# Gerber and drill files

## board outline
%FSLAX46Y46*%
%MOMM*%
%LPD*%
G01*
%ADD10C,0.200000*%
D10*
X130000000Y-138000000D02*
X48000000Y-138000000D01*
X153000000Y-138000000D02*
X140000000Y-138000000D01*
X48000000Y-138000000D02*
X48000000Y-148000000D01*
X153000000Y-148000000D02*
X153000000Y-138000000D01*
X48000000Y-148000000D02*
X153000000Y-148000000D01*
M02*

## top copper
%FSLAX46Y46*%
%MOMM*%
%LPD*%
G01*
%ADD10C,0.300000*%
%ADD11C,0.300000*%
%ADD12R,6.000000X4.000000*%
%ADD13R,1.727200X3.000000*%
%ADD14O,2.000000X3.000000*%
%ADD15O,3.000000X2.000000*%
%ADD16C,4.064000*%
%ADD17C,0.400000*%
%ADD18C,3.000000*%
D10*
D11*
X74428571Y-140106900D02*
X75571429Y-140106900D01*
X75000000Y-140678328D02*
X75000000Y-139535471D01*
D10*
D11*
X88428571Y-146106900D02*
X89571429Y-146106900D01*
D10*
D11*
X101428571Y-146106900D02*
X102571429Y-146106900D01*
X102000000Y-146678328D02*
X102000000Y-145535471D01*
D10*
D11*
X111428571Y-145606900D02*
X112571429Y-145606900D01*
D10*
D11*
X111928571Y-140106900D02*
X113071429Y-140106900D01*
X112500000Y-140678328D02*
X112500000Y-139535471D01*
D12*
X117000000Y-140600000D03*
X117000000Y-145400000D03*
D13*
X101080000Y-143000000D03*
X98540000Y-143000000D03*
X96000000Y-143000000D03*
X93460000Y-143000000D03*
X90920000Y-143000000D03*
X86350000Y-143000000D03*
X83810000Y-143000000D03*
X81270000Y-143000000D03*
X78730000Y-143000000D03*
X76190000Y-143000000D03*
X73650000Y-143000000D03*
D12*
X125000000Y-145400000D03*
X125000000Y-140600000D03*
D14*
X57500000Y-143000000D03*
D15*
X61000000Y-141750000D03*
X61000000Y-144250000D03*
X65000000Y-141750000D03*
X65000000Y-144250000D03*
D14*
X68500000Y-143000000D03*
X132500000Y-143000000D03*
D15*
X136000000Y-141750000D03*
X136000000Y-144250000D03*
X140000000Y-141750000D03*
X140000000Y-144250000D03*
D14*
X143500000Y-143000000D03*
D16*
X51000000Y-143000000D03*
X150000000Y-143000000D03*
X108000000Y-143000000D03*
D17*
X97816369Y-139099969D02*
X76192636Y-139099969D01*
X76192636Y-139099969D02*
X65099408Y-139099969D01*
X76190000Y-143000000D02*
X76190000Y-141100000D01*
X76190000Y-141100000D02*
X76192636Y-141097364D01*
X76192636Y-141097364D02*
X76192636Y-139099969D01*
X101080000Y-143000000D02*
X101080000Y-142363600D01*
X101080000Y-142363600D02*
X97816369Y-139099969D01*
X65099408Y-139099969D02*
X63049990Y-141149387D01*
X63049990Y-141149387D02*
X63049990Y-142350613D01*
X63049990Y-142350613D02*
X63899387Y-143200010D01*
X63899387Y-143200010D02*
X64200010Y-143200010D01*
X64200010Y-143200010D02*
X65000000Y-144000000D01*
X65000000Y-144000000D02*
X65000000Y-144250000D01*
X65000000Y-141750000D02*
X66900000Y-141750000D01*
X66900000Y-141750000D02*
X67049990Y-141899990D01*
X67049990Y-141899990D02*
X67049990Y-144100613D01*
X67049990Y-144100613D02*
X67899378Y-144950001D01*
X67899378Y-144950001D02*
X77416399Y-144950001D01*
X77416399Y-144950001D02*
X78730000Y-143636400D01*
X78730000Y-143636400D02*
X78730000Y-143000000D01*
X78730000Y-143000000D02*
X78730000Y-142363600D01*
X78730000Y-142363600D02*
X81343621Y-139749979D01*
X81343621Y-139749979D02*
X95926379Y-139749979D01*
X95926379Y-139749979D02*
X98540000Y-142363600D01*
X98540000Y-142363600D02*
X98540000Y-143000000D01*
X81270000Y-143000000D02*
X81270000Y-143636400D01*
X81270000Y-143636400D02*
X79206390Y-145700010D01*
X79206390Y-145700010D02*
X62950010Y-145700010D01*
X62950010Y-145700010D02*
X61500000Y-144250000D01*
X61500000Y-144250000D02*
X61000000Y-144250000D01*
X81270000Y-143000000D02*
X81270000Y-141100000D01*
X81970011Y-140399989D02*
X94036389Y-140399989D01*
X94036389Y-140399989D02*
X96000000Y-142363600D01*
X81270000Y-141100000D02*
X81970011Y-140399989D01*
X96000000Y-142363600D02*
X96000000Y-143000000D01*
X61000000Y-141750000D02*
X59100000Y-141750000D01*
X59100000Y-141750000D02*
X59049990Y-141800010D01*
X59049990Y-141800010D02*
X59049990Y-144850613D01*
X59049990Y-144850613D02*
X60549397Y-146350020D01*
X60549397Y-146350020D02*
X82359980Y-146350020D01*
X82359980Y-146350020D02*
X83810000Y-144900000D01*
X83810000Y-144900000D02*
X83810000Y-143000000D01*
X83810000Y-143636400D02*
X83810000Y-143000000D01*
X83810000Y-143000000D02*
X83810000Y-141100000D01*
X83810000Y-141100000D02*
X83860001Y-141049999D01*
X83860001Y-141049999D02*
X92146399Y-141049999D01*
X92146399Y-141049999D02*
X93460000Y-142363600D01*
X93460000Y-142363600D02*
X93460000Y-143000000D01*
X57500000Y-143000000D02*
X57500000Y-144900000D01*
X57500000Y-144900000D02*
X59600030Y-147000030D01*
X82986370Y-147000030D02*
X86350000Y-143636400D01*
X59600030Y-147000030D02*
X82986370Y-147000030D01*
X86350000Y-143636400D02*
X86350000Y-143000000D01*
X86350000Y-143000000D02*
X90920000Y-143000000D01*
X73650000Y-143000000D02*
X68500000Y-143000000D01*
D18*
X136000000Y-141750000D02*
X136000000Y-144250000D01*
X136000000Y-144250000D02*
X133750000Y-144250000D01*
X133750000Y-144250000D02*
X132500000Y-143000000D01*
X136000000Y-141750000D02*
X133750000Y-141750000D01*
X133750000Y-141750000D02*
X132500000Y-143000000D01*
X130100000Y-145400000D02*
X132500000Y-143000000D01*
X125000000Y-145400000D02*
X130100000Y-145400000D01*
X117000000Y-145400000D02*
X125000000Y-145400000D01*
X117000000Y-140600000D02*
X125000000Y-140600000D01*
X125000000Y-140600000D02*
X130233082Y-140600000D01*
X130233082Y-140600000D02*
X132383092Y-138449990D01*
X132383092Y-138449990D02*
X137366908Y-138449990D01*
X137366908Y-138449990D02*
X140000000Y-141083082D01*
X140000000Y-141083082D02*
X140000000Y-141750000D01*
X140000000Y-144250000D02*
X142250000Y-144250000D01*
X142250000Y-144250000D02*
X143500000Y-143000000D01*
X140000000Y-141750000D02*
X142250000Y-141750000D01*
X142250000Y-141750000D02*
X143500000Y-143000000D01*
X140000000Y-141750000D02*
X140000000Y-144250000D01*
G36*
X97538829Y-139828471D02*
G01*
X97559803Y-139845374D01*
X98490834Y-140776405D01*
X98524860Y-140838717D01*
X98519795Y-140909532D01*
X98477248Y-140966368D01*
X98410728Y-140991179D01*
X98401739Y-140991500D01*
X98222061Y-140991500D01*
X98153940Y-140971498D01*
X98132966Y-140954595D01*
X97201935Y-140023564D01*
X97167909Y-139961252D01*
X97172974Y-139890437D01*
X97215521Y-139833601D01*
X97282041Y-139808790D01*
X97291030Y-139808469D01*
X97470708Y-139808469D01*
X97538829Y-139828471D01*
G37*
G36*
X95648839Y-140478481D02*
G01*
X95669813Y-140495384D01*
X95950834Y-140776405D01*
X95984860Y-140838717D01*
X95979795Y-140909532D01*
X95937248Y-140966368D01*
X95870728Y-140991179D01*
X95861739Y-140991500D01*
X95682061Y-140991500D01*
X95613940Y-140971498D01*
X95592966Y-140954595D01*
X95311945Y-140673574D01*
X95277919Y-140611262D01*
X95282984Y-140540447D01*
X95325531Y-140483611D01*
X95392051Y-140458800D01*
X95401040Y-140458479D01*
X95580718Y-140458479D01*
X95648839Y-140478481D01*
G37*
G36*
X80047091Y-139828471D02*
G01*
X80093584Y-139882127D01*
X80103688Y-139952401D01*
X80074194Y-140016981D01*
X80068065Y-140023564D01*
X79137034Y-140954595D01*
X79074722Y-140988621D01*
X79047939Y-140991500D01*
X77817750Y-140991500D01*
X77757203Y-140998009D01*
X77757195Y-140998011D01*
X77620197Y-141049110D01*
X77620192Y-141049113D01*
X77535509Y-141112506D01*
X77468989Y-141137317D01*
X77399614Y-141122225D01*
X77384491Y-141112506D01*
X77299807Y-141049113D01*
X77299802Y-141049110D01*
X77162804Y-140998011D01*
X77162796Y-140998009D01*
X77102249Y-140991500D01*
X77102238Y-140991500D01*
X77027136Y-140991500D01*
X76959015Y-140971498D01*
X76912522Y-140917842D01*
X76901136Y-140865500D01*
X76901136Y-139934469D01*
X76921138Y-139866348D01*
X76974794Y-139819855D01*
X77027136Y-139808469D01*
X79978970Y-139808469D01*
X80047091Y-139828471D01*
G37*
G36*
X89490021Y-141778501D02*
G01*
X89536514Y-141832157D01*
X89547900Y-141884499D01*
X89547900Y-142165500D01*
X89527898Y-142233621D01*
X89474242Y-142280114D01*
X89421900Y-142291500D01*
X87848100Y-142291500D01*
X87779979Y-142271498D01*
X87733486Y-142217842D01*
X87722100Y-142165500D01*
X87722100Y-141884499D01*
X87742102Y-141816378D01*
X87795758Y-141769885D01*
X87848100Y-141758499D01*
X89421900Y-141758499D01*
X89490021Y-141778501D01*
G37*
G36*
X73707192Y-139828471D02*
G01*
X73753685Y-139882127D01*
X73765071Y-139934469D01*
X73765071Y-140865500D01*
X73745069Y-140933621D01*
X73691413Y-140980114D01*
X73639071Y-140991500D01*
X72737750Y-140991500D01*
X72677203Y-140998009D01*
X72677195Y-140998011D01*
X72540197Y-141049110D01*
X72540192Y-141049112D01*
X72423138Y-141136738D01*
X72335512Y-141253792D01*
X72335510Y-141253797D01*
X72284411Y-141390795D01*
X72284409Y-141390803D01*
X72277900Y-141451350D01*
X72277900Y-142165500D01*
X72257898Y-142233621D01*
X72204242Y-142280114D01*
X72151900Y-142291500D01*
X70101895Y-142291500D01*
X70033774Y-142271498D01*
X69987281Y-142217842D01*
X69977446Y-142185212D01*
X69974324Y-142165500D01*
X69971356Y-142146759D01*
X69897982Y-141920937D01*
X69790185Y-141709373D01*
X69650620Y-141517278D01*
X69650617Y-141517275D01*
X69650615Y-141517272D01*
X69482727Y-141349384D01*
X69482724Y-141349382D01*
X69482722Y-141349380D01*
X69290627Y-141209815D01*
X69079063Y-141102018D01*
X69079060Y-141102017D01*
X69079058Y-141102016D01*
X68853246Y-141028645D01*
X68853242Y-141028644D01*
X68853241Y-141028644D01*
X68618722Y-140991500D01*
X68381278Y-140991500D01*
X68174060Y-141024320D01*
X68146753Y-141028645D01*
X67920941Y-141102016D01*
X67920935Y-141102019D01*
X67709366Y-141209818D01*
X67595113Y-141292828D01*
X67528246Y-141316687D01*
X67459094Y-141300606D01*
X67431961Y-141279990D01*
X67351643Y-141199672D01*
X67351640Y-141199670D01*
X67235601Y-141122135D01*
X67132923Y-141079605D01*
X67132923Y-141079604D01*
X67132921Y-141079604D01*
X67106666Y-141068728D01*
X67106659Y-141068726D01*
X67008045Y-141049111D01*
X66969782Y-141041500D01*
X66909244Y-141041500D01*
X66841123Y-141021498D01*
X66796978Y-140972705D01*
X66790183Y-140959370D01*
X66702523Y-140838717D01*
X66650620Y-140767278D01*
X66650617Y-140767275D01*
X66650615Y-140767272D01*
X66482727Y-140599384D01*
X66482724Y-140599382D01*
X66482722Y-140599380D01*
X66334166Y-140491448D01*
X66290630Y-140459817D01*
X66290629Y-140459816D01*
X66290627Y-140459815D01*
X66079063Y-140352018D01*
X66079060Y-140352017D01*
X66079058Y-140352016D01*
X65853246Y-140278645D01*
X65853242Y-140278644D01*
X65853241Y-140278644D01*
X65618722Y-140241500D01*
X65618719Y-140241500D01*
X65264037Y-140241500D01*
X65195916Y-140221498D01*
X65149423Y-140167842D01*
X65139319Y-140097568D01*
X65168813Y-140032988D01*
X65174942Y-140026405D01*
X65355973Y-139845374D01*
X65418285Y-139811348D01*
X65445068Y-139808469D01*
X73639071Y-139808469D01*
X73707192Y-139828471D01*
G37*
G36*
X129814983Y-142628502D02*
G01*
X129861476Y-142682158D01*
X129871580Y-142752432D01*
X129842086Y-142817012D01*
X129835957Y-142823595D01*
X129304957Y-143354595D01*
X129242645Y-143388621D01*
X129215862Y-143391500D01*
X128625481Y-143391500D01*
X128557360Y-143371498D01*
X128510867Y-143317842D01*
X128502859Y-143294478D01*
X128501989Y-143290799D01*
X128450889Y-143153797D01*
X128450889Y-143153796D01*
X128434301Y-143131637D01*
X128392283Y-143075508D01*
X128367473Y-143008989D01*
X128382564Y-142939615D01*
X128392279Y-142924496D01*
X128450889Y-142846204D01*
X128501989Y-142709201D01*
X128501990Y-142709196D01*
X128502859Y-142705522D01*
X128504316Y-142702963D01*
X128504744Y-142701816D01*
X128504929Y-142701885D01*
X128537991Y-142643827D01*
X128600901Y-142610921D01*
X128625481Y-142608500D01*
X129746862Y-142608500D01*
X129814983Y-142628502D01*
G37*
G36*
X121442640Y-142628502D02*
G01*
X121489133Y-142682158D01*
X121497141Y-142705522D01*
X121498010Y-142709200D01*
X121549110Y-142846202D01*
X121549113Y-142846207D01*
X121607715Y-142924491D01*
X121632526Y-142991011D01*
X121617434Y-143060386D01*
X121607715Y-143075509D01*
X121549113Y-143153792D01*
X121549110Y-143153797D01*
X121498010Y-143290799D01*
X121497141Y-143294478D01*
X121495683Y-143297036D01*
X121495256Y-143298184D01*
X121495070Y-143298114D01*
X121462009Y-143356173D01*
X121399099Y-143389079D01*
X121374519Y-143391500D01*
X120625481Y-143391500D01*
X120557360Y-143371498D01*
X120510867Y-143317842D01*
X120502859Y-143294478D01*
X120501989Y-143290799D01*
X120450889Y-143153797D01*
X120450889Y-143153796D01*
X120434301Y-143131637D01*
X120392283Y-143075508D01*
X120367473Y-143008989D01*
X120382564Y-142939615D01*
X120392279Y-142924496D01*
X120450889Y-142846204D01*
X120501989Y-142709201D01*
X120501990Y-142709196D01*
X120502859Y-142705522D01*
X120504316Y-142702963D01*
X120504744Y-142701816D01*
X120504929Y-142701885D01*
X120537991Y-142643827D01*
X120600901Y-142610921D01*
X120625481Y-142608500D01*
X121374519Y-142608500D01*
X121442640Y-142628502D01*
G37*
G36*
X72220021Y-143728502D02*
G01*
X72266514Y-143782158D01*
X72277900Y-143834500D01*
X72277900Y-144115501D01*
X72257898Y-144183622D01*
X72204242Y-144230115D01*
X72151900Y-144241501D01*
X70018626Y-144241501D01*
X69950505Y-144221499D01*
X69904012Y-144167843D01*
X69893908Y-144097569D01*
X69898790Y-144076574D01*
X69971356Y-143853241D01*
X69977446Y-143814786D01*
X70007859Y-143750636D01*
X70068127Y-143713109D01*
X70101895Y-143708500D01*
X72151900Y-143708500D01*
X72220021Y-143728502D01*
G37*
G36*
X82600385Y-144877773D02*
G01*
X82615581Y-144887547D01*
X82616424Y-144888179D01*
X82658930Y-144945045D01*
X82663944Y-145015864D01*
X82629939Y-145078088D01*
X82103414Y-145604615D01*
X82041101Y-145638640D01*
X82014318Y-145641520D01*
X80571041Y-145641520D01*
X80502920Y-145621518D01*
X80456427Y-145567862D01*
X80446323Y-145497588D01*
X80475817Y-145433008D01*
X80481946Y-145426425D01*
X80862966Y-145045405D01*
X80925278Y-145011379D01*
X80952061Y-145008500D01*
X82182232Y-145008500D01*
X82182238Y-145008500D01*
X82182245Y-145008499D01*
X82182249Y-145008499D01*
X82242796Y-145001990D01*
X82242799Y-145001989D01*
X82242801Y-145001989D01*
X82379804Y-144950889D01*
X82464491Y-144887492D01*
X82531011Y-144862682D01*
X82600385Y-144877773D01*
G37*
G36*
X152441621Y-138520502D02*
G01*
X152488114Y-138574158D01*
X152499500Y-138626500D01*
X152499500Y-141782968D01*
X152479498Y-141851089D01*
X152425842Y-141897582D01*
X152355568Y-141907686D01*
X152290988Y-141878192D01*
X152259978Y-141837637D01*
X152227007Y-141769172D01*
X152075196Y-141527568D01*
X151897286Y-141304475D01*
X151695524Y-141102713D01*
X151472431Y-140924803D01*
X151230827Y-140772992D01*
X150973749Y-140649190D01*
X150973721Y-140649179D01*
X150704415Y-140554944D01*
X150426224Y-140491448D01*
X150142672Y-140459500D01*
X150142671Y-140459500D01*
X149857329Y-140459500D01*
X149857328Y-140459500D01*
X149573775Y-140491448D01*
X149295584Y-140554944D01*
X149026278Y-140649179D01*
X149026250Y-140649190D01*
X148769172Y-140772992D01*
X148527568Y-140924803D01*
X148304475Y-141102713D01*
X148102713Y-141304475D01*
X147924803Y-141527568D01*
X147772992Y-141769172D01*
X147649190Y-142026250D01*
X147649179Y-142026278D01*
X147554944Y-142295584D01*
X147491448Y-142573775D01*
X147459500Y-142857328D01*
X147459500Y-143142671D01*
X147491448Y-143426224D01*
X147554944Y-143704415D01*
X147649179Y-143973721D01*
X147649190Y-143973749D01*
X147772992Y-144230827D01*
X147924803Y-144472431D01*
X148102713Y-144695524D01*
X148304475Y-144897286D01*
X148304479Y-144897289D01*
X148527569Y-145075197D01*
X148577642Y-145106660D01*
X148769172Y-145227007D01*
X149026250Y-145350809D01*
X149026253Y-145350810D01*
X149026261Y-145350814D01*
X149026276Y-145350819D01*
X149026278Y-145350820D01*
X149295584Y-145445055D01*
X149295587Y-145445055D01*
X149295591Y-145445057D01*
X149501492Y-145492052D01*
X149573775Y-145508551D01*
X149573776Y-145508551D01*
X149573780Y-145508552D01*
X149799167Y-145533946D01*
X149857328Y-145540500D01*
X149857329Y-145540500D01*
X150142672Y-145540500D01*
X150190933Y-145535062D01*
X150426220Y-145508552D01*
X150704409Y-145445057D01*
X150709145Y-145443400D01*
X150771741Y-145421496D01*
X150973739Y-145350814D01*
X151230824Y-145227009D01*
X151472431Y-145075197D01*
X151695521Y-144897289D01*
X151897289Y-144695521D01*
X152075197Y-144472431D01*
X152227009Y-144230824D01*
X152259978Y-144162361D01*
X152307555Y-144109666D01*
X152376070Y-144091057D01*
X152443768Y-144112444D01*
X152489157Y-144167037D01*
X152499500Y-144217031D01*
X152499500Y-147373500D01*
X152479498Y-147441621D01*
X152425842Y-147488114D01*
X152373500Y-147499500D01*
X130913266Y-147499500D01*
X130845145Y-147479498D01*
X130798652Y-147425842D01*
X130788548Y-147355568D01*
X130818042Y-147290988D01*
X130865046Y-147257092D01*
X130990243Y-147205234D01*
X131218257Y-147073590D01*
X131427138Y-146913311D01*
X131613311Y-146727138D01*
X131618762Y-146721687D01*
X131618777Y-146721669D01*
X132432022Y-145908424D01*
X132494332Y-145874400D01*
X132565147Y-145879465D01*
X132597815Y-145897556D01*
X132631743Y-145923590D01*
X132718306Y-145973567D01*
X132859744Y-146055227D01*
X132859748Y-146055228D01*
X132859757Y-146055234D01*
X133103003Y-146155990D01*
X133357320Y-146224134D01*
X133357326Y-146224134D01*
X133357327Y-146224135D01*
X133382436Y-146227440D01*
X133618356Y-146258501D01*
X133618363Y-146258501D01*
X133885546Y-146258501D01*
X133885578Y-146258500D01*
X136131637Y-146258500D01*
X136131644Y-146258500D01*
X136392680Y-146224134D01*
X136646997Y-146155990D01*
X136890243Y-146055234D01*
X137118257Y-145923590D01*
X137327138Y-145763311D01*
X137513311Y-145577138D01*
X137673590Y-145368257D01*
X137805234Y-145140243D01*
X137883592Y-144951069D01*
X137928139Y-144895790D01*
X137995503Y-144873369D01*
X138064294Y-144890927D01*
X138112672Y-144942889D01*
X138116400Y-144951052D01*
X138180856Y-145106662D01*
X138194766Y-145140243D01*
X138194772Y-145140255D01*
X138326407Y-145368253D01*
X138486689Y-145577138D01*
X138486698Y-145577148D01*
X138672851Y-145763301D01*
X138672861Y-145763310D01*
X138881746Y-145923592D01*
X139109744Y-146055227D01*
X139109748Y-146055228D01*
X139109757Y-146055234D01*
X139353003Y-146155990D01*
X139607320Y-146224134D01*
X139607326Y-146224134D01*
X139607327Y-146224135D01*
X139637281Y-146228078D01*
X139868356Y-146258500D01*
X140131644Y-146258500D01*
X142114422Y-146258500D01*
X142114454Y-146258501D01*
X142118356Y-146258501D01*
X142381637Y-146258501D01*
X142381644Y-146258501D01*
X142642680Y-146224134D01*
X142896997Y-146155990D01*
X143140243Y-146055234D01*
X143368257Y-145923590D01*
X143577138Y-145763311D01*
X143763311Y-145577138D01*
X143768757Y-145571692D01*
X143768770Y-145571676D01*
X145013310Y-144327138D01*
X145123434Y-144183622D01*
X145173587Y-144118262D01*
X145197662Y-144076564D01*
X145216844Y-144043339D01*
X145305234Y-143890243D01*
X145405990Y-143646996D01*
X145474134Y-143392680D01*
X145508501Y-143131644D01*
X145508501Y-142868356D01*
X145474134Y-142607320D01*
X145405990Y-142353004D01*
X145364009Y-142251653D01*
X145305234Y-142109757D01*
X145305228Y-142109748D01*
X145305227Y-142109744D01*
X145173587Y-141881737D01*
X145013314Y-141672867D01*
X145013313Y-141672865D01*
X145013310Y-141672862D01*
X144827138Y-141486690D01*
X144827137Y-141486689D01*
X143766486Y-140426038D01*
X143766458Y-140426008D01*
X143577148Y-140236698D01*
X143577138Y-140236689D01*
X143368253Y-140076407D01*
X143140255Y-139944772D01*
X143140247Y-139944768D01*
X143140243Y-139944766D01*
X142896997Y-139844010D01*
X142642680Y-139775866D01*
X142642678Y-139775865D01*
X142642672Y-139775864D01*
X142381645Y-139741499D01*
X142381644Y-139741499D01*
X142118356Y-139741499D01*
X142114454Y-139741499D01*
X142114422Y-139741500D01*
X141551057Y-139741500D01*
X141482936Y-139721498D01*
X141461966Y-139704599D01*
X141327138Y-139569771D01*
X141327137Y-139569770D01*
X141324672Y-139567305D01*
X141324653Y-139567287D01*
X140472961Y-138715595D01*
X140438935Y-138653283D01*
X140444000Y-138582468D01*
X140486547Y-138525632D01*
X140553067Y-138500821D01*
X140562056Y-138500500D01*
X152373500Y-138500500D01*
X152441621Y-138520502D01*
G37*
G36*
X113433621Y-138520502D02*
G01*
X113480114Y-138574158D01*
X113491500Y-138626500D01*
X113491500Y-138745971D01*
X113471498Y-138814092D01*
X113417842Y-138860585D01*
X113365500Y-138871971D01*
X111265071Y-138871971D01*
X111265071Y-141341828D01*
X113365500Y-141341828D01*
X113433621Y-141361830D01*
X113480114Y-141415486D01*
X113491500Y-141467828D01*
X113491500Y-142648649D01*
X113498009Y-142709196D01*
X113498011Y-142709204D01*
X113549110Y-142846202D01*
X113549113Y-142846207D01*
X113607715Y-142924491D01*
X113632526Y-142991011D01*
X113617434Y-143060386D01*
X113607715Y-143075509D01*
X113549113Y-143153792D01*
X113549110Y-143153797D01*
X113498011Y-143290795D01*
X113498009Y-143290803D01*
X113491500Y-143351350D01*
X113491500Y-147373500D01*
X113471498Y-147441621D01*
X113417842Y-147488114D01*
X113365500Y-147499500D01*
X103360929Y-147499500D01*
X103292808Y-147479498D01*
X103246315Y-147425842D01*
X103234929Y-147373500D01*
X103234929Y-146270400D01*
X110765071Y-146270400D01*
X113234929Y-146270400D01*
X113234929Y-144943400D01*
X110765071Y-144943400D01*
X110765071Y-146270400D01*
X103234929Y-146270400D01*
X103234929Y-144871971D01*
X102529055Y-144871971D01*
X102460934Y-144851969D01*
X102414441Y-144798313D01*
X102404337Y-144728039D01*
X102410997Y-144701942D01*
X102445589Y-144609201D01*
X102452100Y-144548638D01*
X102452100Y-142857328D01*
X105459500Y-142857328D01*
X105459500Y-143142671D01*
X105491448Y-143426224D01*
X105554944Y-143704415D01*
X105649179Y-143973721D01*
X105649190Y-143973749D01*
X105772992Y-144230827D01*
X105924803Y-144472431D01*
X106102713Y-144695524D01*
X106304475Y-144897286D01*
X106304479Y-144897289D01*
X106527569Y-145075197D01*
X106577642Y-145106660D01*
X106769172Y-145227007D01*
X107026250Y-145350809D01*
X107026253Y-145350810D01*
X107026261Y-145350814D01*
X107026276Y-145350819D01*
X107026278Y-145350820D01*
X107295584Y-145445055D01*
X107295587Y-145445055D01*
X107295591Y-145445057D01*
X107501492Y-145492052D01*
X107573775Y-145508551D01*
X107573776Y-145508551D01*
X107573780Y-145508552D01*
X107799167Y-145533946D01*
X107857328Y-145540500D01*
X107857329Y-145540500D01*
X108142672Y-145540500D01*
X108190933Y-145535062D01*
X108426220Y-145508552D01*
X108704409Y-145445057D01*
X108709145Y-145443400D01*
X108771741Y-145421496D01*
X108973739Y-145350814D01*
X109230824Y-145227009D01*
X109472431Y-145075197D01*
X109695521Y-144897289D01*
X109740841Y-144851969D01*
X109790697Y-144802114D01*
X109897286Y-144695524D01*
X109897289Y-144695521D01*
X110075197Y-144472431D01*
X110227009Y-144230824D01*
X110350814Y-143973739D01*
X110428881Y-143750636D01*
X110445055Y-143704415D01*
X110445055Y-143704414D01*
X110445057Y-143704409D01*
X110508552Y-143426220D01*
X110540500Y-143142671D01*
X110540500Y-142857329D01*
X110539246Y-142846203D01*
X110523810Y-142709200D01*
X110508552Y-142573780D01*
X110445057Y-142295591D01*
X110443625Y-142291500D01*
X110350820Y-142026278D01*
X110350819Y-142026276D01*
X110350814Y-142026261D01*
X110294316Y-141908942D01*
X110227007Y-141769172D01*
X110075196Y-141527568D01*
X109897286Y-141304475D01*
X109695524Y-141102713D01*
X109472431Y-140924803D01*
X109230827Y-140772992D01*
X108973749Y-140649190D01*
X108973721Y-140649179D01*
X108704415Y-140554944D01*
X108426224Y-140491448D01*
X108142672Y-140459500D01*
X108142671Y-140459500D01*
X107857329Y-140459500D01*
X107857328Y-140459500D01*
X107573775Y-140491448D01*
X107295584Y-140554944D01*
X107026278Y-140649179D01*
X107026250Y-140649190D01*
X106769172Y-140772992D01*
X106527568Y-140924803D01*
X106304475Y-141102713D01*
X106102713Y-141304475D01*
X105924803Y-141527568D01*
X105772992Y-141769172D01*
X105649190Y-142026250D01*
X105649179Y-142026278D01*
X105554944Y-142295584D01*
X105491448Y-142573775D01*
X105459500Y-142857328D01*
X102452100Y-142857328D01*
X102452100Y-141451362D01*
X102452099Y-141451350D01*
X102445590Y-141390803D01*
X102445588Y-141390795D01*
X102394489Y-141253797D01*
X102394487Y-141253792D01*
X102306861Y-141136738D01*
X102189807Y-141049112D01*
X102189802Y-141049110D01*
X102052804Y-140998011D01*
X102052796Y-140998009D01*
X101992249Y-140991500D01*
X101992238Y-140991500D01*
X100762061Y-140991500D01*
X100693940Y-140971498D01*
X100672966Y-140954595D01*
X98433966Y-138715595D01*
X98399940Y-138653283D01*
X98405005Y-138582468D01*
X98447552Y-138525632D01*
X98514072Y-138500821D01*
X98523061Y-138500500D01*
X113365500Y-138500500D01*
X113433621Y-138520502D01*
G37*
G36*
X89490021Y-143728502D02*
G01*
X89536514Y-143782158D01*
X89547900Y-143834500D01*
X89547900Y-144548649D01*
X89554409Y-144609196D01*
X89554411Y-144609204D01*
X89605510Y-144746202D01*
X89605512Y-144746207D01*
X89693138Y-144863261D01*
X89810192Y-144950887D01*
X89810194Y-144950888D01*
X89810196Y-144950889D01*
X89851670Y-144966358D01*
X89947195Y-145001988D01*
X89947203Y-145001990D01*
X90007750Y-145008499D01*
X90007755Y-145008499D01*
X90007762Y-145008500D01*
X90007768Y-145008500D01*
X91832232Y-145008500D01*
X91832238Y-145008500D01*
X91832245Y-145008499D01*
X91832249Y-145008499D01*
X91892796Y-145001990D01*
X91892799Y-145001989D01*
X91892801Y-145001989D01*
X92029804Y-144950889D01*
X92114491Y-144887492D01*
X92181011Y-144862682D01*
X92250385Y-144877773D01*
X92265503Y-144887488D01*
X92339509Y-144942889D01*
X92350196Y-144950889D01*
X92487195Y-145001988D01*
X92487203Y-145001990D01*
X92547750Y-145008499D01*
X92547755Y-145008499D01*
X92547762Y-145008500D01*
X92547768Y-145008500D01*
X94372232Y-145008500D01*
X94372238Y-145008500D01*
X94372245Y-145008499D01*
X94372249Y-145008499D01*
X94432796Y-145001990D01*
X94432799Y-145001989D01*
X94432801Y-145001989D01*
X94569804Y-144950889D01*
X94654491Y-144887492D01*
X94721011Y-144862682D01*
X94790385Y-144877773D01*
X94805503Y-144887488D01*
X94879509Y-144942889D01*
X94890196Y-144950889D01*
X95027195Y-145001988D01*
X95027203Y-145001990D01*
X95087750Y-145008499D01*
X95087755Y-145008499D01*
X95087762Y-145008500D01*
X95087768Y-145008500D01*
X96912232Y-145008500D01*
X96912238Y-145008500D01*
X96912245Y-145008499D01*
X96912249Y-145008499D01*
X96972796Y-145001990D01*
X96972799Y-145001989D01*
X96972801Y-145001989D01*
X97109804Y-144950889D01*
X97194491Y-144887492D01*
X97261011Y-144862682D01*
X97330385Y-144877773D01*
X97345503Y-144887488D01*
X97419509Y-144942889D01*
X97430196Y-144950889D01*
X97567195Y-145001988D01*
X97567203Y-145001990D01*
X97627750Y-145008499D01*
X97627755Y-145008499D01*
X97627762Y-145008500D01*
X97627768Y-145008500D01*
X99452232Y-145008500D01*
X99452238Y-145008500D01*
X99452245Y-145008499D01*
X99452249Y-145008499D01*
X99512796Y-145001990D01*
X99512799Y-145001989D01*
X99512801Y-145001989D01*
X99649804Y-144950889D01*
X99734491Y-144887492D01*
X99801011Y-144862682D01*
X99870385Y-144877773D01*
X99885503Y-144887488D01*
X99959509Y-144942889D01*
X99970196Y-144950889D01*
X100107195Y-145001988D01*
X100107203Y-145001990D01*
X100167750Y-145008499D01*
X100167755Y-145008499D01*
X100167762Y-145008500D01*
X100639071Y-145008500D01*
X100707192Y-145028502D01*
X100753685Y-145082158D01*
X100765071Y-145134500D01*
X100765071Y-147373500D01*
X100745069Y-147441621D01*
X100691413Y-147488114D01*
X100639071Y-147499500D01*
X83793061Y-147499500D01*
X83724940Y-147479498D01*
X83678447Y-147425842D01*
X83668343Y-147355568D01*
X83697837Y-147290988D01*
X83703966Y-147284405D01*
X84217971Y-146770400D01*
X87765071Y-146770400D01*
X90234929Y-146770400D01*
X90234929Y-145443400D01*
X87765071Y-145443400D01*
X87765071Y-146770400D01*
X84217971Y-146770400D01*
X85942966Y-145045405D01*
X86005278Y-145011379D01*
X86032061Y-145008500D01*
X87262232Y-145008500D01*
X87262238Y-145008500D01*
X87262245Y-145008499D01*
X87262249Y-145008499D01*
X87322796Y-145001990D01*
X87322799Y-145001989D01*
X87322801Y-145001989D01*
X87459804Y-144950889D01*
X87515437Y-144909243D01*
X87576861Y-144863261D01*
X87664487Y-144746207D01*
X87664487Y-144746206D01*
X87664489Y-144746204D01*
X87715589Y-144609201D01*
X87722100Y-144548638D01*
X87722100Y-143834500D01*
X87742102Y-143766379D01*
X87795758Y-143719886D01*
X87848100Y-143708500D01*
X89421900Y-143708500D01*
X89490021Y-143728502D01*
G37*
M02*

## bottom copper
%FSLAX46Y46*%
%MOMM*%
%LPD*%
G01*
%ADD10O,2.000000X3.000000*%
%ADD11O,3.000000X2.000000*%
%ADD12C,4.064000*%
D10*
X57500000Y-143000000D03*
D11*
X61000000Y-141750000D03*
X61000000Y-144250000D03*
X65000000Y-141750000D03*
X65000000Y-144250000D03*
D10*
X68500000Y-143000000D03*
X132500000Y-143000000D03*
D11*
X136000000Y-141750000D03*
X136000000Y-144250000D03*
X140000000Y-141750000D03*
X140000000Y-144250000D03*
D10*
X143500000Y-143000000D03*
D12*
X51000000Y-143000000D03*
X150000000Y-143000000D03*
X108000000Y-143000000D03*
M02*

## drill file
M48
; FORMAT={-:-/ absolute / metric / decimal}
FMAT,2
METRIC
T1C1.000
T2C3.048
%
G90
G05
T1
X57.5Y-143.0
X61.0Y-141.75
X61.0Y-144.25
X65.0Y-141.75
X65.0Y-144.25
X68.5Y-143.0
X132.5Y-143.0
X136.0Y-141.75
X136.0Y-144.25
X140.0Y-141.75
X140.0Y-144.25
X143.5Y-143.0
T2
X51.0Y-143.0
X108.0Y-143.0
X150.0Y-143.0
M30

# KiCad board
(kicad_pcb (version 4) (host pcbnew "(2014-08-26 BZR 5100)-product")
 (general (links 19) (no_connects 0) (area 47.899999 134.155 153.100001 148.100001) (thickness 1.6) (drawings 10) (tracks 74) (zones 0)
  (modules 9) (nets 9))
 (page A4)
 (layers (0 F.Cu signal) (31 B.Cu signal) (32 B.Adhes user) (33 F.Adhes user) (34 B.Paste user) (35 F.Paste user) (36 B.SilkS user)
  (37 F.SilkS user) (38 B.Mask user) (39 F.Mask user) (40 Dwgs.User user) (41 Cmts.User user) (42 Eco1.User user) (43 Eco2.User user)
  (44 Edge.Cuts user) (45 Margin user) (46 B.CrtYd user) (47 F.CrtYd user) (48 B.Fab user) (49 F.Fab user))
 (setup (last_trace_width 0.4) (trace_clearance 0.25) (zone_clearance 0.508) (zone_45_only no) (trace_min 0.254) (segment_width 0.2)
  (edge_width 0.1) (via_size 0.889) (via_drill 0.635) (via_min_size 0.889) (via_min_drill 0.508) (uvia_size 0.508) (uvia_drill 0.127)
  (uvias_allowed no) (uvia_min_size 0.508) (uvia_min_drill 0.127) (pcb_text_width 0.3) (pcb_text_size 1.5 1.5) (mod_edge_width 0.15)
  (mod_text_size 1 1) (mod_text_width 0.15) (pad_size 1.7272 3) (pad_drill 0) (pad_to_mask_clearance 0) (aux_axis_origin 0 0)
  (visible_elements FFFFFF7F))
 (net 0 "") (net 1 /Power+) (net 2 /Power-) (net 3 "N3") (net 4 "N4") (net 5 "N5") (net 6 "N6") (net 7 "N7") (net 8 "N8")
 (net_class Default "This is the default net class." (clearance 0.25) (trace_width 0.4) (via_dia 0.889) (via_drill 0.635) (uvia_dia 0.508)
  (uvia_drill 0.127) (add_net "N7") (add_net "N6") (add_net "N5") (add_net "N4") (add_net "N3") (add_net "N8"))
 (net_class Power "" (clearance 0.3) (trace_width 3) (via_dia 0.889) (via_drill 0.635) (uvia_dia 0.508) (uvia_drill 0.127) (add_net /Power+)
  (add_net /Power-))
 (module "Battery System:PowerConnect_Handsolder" (layer F.Cu) (at 117 143)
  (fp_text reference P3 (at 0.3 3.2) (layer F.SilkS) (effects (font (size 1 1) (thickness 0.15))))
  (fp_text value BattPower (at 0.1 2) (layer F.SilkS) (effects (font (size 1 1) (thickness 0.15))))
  (pad 1 smd rect (at 0 -2.4) (size 6 4) (layers F.Cu F.Paste F.Mask) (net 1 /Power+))
  (pad 2 smd rect (at 0 2.4) (size 6 4) (layers F.Cu F.Paste F.Mask) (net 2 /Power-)))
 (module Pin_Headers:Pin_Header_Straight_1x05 (layer F.Cu) (at 96 143 180)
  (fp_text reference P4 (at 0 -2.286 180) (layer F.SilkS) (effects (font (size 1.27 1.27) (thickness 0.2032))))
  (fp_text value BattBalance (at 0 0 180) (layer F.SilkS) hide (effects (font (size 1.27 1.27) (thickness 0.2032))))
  (pad 1 smd rect (at -5.08 0) (size 1.7272 3) (layers F.Cu F.Paste F.Mask) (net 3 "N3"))
  (pad 2 smd rect (at -2.54 0) (size 1.7272 3) (layers F.Cu F.Paste F.Mask) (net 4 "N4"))
  (pad 3 smd rect (at 0 0) (size 1.7272 3) (layers F.Cu F.Paste F.Mask) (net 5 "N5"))
  (pad 4 smd rect (at 2.54 0) (size 1.7272 3) (layers F.Cu F.Paste F.Mask) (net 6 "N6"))
  (pad 5 smd rect (at 5.08 0) (size 1.7272 3) (layers F.Cu F.Paste F.Mask) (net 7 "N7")))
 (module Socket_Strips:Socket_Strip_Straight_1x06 (layer F.Cu) (at 80 143)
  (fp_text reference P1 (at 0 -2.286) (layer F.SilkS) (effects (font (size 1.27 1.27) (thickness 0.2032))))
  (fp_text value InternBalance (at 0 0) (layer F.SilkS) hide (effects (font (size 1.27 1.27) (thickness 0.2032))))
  (pad 1 smd rect (at 6.35 0 180) (size 1.7272 3) (layers F.Cu F.Paste F.Mask) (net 7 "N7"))
  (pad 2 smd rect (at 3.81 0 180) (size 1.7272 3) (layers F.Cu F.Paste F.Mask) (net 6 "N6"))
  (pad 3 smd rect (at 1.27 0 180) (size 1.7272 3) (layers F.Cu F.Paste F.Mask) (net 5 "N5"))
  (pad 4 smd rect (at -1.27 0 180) (size 1.7272 3) (layers F.Cu F.Paste F.Mask) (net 4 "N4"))
  (pad 5 smd rect (at -3.81 0 180) (size 1.7272 3) (layers F.Cu F.Paste F.Mask) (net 3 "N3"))
  (pad 6 smd rect (at -6.35 0 180) (size 1.7272 3) (layers F.Cu F.Paste F.Mask) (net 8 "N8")))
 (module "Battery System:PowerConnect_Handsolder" (layer F.Cu) (at 125 143 180)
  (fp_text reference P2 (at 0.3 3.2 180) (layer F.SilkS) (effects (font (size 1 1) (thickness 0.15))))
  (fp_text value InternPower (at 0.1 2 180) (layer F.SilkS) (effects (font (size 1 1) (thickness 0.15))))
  (pad 1 smd rect (at 0 -2.4 180) (size 6 4) (layers F.Cu F.Paste F.Mask) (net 2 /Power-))
  (pad 2 smd rect (at 0 2.4 180) (size 6 4) (layers F.Cu F.Paste F.Mask) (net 1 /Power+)))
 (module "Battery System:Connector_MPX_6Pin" (layer B.Cu) (at 63 143)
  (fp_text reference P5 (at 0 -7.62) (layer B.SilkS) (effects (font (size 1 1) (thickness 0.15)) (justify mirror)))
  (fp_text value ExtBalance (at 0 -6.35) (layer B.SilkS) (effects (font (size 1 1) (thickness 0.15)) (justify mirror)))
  (pad 1 thru_hole oval (at -5.5 0 180) (size 2 3) (drill 1) (layers *.Cu *.Mask B.SilkS) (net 7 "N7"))
  (pad 2 thru_hole oval (at -2 -1.25 180) (size 3 2) (drill 1) (layers *.Cu *.Mask B.SilkS) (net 6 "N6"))
  (pad 3 thru_hole oval (at -2 1.25 180) (size 3 2) (drill 1) (layers *.Cu *.Mask B.SilkS) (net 5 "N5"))
  (pad 4 thru_hole oval (at 2 -1.25 180) (size 3 2) (drill 1) (layers *.Cu *.Mask B.SilkS) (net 4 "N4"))
  (pad 5 thru_hole oval (at 2 1.25 180) (size 3 2) (drill 1) (layers *.Cu *.Mask B.SilkS) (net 3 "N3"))
  (pad 6 thru_hole oval (at 5.5 0 180) (size 2 3) (drill 1) (layers *.Cu *.Mask B.SilkS) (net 8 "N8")))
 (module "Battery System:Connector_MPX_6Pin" (layer B.Cu) (at 138 143)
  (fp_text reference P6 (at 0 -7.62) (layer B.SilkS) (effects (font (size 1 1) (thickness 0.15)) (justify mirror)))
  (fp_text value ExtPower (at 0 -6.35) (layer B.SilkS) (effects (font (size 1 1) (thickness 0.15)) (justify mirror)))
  (pad 1 thru_hole oval (at -5.5 0 180) (size 2 3) (drill 1) (layers *.Cu *.Mask B.SilkS) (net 2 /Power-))
  (pad 2 thru_hole oval (at -2 -1.25 180) (size 3 2) (drill 1) (layers *.Cu *.Mask B.SilkS) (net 2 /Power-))
  (pad 3 thru_hole oval (at -2 1.25 180) (size 3 2) (drill 1) (layers *.Cu *.Mask B.SilkS) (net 2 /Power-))
  (pad 4 thru_hole oval (at 2 -1.25 180) (size 3 2) (drill 1) (layers *.Cu *.Mask B.SilkS) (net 1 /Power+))
  (pad 5 thru_hole oval (at 2 1.25 180) (size 3 2) (drill 1) (layers *.Cu *.Mask B.SilkS) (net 1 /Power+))
  (pad 6 thru_hole oval (at 5.5 0 180) (size 2 3) (drill 1) (layers *.Cu *.Mask B.SilkS) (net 1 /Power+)))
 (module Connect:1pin (layer F.Cu) (at 51 143)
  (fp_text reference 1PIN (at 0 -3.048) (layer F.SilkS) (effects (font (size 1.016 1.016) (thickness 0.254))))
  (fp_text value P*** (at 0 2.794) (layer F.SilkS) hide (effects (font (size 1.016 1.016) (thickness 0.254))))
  (pad 1 thru_hole circle (at 0 0) (size 4.064 4.064) (drill 3.048) (layers *.Cu *.Mask F.SilkS)))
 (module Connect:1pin (layer F.Cu) (at 150 143)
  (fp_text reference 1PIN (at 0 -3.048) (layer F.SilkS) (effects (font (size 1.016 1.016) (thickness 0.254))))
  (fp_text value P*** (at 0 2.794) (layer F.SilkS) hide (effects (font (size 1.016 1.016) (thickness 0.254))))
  (pad 1 thru_hole circle (at 0 0) (size 4.064 4.064) (drill 3.048) (layers *.Cu *.Mask F.SilkS)))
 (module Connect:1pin (layer F.Cu) (at 108 143)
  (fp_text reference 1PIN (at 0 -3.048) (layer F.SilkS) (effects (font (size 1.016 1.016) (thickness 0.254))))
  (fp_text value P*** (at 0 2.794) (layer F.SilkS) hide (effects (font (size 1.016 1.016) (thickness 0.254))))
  (pad 1 thru_hole circle (at 0 0) (size 4.064 4.064) (drill 3.048) (layers *.Cu *.Mask F.SilkS)))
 (gr_line (start 130 138) (end 48 138) (layer Edge.Cuts) (width 0.2))
 (gr_line (start 153 138) (end 140 138) (layer Edge.Cuts) (width 0.2))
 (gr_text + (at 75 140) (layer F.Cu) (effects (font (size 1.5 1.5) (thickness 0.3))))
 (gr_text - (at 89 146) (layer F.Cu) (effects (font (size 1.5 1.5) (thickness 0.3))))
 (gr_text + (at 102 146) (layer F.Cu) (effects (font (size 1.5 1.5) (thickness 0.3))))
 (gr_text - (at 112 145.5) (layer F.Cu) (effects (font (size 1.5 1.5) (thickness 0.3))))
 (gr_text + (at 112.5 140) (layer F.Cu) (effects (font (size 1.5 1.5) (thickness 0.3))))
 (gr_line (start 48 138) (end 48 148) (layer Edge.Cuts) (width 0.2))
 (gr_line (start 153 148) (end 153 138) (layer Edge.Cuts) (width 0.2))
 (gr_line (start 48 148) (end 153 148) (layer Edge.Cuts) (width 0.2))
 (segment (start 97.816369 139.099969) (end 76.192636 139.099969) (width 0.4) (layer F.Cu) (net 3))
 (segment (start 76.192636 139.099969) (end 65.099408 139.099969) (width 0.4) (layer F.Cu) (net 3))
 (segment (start 76.19 143) (end 76.19 141.1) (width 0.4) (layer F.Cu) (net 3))
 (segment (start 76.19 141.1) (end 76.192636 141.097364) (width 0.4) (layer F.Cu) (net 3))
 (segment (start 76.192636 141.097364) (end 76.192636 139.099969) (width 0.4) (layer F.Cu) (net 3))
 (segment (start 101.08 143) (end 101.08 142.3636) (width 0.4) (layer F.Cu) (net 3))
 (segment (start 101.08 142.3636) (end 97.816369 139.099969) (width 0.4) (layer F.Cu) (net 3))
 (segment (start 65.099408 139.099969) (end 63.04999 141.149387) (width 0.4) (layer F.Cu) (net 3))
 (segment (start 63.04999 141.149387) (end 63.04999 142.350613) (width 0.4) (layer F.Cu) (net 3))
 (segment (start 63.04999 142.350613) (end 63.899387 143.20001) (width 0.4) (layer F.Cu) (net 3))
 (segment (start 63.899387 143.20001) (end 64.20001 143.20001) (width 0.4) (layer F.Cu) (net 3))
 (segment (start 64.20001 143.20001) (end 65 144) (width 0.4) (layer F.Cu) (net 3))
 (segment (start 65 144) (end 65 144.25) (width 0.4) (layer F.Cu) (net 3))
 (segment (start 65 141.75) (end 66.9 141.75) (width 0.4) (layer F.Cu) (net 4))
 (segment (start 66.9 141.75) (end 67.04999 141.89999) (width 0.4) (layer F.Cu) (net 4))
 (segment (start 67.04999 141.89999) (end 67.04999 144.100613) (width 0.4) (layer F.Cu) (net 4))
 (segment (start 67.04999 144.100613) (end 67.899378 144.950001) (width 0.4) (layer F.Cu) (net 4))
 (segment (start 67.899378 144.950001) (end 77.416399 144.950001) (width 0.4) (layer F.Cu) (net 4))
 (segment (start 77.416399 144.950001) (end 78.73 143.6364) (width 0.4) (layer F.Cu) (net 4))
 (segment (start 78.73 143.6364) (end 78.73 143) (width 0.4) (layer F.Cu) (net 4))
 (segment (start 78.73 143) (end 78.73 142.3636) (width 0.4) (layer F.Cu) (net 4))
 (segment (start 78.73 142.3636) (end 81.343621 139.749979) (width 0.4) (layer F.Cu) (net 4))
 (segment (start 81.343621 139.749979) (end 95.926379 139.749979) (width 0.4) (layer F.Cu) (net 4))
 (segment (start 95.926379 139.749979) (end 98.54 142.3636) (width 0.4) (layer F.Cu) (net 4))
 (segment (start 98.54 142.3636) (end 98.54 143) (width 0.4) (layer F.Cu) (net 4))
 (segment (start 81.27 143) (end 81.27 143.6364) (width 0.4) (layer F.Cu) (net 5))
 (segment (start 81.27 143.6364) (end 79.20639 145.70001) (width 0.4) (layer F.Cu) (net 5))
 (segment (start 79.20639 145.70001) (end 62.95001 145.70001) (width 0.4) (layer F.Cu) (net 5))
 (segment (start 62.95001 145.70001) (end 61.5 144.25) (width 0.4) (layer F.Cu) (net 5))
 (segment (start 61.5 144.25) (end 61 144.25) (width 0.4) (layer F.Cu) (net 5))
 (segment (start 81.27 143) (end 81.27 141.1) (width 0.4) (layer F.Cu) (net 5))
 (segment (start 81.970011 140.399989) (end 94.036389 140.399989) (width 0.4) (layer F.Cu) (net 5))
 (segment (start 94.036389 140.399989) (end 96 142.3636) (width 0.4) (layer F.Cu) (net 5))
 (segment (start 81.27 141.1) (end 81.970011 140.399989) (width 0.4) (layer F.Cu) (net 5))
 (segment (start 96 142.3636) (end 96 143) (width 0.4) (layer F.Cu) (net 5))
 (segment (start 61 141.75) (end 59.1 141.75) (width 0.4) (layer F.Cu) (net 6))
 (segment (start 59.1 141.75) (end 59.04999 141.80001) (width 0.4) (layer F.Cu) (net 6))
 (segment (start 59.04999 141.80001) (end 59.04999 144.850613) (width 0.4) (layer F.Cu) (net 6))
 (segment (start 59.04999 144.850613) (end 60.549397 146.35002) (width 0.4) (layer F.Cu) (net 6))
 (segment (start 60.549397 146.35002) (end 82.35998 146.35002) (width 0.4) (layer F.Cu) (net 6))
 (segment (start 82.35998 146.35002) (end 83.81 144.9) (width 0.4) (layer F.Cu) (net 6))
 (segment (start 83.81 144.9) (end 83.81 143) (width 0.4) (layer F.Cu) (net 6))
 (segment (start 83.81 143.6364) (end 83.81 143) (width 0.4) (layer F.Cu) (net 6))
 (segment (start 83.81 143) (end 83.81 141.1) (width 0.4) (layer F.Cu) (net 6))
 (segment (start 83.81 141.1) (end 83.860001 141.049999) (width 0.4) (layer F.Cu) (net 6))
 (segment (start 83.860001 141.049999) (end 92.146399 141.049999) (width 0.4) (layer F.Cu) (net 6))
 (segment (start 92.146399 141.049999) (end 93.46 142.3636) (width 0.4) (layer F.Cu) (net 6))
 (segment (start 93.46 142.3636) (end 93.46 143) (width 0.4) (layer F.Cu) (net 6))
 (segment (start 57.5 143) (end 57.5 144.9) (width 0.4) (layer F.Cu) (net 7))
 (segment (start 57.5 144.9) (end 59.60003 147.00003) (width 0.4) (layer F.Cu) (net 7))
 (segment (start 82.98637 147.00003) (end 86.35 143.6364) (width 0.4) (layer F.Cu) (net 7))
 (segment (start 59.60003 147.00003) (end 82.98637 147.00003) (width 0.4) (layer F.Cu) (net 7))
 (segment (start 86.35 143.6364) (end 86.35 143) (width 0.4) (layer F.Cu) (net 7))
 (segment (start 86.35 143) (end 90.92 143) (width 0.4) (layer F.Cu) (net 7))
 (segment (start 73.65 143) (end 68.5 143) (width 0.4) (layer F.Cu) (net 8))
 (segment (start 136 141.75) (end 136 144.25) (width 3) (layer F.Cu) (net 2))
 (segment (start 136 144.25) (end 133.75 144.25) (width 3) (layer F.Cu) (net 2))
 (segment (start 133.75 144.25) (end 132.5 143) (width 3) (layer F.Cu) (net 2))
 (segment (start 136 141.75) (end 133.75 141.75) (width 3) (layer F.Cu) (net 2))
 (segment (start 133.75 141.75) (end 132.5 143) (width 3) (layer F.Cu) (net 2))
 (segment (start 130.1 145.4) (end 132.5 143) (width 3) (layer F.Cu) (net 2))
 (segment (start 125 145.4) (end 130.1 145.4) (width 3) (layer F.Cu) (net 2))
 (segment (start 117 145.4) (end 125 145.4) (width 3) (layer F.Cu) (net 2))
 (segment (start 117 140.6) (end 125 140.6) (width 3) (layer F.Cu) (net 1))
 (segment (start 125 140.6) (end 130.233082 140.6) (width 3) (layer F.Cu) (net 1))
 (segment (start 130.233082 140.6) (end 132.383092 138.44999) (width 3) (layer F.Cu) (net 1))
 (segment (start 132.383092 138.44999) (end 137.366908 138.44999) (width 3) (layer F.Cu) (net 1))
 (segment (start 137.366908 138.44999) (end 140 141.083082) (width 3) (layer F.Cu) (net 1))
 (segment (start 140 141.083082) (end 140 141.75) (width 3) (layer F.Cu) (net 1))
 (segment (start 140 144.25) (end 142.25 144.25) (width 3) (layer F.Cu) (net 1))
 (segment (start 142.25 144.25) (end 143.5 143) (width 3) (layer F.Cu) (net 1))
 (segment (start 140 141.75) (end 142.25 141.75) (width 3) (layer F.Cu) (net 1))
 (segment (start 142.25 141.75) (end 143.5 143) (width 3) (layer F.Cu) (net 1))
 (segment (start 140 141.75) (end 140 144.25) (width 3) (layer F.Cu) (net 1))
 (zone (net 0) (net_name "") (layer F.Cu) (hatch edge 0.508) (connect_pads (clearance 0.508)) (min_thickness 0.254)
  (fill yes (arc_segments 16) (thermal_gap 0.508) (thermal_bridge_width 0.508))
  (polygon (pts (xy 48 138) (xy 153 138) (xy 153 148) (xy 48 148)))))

